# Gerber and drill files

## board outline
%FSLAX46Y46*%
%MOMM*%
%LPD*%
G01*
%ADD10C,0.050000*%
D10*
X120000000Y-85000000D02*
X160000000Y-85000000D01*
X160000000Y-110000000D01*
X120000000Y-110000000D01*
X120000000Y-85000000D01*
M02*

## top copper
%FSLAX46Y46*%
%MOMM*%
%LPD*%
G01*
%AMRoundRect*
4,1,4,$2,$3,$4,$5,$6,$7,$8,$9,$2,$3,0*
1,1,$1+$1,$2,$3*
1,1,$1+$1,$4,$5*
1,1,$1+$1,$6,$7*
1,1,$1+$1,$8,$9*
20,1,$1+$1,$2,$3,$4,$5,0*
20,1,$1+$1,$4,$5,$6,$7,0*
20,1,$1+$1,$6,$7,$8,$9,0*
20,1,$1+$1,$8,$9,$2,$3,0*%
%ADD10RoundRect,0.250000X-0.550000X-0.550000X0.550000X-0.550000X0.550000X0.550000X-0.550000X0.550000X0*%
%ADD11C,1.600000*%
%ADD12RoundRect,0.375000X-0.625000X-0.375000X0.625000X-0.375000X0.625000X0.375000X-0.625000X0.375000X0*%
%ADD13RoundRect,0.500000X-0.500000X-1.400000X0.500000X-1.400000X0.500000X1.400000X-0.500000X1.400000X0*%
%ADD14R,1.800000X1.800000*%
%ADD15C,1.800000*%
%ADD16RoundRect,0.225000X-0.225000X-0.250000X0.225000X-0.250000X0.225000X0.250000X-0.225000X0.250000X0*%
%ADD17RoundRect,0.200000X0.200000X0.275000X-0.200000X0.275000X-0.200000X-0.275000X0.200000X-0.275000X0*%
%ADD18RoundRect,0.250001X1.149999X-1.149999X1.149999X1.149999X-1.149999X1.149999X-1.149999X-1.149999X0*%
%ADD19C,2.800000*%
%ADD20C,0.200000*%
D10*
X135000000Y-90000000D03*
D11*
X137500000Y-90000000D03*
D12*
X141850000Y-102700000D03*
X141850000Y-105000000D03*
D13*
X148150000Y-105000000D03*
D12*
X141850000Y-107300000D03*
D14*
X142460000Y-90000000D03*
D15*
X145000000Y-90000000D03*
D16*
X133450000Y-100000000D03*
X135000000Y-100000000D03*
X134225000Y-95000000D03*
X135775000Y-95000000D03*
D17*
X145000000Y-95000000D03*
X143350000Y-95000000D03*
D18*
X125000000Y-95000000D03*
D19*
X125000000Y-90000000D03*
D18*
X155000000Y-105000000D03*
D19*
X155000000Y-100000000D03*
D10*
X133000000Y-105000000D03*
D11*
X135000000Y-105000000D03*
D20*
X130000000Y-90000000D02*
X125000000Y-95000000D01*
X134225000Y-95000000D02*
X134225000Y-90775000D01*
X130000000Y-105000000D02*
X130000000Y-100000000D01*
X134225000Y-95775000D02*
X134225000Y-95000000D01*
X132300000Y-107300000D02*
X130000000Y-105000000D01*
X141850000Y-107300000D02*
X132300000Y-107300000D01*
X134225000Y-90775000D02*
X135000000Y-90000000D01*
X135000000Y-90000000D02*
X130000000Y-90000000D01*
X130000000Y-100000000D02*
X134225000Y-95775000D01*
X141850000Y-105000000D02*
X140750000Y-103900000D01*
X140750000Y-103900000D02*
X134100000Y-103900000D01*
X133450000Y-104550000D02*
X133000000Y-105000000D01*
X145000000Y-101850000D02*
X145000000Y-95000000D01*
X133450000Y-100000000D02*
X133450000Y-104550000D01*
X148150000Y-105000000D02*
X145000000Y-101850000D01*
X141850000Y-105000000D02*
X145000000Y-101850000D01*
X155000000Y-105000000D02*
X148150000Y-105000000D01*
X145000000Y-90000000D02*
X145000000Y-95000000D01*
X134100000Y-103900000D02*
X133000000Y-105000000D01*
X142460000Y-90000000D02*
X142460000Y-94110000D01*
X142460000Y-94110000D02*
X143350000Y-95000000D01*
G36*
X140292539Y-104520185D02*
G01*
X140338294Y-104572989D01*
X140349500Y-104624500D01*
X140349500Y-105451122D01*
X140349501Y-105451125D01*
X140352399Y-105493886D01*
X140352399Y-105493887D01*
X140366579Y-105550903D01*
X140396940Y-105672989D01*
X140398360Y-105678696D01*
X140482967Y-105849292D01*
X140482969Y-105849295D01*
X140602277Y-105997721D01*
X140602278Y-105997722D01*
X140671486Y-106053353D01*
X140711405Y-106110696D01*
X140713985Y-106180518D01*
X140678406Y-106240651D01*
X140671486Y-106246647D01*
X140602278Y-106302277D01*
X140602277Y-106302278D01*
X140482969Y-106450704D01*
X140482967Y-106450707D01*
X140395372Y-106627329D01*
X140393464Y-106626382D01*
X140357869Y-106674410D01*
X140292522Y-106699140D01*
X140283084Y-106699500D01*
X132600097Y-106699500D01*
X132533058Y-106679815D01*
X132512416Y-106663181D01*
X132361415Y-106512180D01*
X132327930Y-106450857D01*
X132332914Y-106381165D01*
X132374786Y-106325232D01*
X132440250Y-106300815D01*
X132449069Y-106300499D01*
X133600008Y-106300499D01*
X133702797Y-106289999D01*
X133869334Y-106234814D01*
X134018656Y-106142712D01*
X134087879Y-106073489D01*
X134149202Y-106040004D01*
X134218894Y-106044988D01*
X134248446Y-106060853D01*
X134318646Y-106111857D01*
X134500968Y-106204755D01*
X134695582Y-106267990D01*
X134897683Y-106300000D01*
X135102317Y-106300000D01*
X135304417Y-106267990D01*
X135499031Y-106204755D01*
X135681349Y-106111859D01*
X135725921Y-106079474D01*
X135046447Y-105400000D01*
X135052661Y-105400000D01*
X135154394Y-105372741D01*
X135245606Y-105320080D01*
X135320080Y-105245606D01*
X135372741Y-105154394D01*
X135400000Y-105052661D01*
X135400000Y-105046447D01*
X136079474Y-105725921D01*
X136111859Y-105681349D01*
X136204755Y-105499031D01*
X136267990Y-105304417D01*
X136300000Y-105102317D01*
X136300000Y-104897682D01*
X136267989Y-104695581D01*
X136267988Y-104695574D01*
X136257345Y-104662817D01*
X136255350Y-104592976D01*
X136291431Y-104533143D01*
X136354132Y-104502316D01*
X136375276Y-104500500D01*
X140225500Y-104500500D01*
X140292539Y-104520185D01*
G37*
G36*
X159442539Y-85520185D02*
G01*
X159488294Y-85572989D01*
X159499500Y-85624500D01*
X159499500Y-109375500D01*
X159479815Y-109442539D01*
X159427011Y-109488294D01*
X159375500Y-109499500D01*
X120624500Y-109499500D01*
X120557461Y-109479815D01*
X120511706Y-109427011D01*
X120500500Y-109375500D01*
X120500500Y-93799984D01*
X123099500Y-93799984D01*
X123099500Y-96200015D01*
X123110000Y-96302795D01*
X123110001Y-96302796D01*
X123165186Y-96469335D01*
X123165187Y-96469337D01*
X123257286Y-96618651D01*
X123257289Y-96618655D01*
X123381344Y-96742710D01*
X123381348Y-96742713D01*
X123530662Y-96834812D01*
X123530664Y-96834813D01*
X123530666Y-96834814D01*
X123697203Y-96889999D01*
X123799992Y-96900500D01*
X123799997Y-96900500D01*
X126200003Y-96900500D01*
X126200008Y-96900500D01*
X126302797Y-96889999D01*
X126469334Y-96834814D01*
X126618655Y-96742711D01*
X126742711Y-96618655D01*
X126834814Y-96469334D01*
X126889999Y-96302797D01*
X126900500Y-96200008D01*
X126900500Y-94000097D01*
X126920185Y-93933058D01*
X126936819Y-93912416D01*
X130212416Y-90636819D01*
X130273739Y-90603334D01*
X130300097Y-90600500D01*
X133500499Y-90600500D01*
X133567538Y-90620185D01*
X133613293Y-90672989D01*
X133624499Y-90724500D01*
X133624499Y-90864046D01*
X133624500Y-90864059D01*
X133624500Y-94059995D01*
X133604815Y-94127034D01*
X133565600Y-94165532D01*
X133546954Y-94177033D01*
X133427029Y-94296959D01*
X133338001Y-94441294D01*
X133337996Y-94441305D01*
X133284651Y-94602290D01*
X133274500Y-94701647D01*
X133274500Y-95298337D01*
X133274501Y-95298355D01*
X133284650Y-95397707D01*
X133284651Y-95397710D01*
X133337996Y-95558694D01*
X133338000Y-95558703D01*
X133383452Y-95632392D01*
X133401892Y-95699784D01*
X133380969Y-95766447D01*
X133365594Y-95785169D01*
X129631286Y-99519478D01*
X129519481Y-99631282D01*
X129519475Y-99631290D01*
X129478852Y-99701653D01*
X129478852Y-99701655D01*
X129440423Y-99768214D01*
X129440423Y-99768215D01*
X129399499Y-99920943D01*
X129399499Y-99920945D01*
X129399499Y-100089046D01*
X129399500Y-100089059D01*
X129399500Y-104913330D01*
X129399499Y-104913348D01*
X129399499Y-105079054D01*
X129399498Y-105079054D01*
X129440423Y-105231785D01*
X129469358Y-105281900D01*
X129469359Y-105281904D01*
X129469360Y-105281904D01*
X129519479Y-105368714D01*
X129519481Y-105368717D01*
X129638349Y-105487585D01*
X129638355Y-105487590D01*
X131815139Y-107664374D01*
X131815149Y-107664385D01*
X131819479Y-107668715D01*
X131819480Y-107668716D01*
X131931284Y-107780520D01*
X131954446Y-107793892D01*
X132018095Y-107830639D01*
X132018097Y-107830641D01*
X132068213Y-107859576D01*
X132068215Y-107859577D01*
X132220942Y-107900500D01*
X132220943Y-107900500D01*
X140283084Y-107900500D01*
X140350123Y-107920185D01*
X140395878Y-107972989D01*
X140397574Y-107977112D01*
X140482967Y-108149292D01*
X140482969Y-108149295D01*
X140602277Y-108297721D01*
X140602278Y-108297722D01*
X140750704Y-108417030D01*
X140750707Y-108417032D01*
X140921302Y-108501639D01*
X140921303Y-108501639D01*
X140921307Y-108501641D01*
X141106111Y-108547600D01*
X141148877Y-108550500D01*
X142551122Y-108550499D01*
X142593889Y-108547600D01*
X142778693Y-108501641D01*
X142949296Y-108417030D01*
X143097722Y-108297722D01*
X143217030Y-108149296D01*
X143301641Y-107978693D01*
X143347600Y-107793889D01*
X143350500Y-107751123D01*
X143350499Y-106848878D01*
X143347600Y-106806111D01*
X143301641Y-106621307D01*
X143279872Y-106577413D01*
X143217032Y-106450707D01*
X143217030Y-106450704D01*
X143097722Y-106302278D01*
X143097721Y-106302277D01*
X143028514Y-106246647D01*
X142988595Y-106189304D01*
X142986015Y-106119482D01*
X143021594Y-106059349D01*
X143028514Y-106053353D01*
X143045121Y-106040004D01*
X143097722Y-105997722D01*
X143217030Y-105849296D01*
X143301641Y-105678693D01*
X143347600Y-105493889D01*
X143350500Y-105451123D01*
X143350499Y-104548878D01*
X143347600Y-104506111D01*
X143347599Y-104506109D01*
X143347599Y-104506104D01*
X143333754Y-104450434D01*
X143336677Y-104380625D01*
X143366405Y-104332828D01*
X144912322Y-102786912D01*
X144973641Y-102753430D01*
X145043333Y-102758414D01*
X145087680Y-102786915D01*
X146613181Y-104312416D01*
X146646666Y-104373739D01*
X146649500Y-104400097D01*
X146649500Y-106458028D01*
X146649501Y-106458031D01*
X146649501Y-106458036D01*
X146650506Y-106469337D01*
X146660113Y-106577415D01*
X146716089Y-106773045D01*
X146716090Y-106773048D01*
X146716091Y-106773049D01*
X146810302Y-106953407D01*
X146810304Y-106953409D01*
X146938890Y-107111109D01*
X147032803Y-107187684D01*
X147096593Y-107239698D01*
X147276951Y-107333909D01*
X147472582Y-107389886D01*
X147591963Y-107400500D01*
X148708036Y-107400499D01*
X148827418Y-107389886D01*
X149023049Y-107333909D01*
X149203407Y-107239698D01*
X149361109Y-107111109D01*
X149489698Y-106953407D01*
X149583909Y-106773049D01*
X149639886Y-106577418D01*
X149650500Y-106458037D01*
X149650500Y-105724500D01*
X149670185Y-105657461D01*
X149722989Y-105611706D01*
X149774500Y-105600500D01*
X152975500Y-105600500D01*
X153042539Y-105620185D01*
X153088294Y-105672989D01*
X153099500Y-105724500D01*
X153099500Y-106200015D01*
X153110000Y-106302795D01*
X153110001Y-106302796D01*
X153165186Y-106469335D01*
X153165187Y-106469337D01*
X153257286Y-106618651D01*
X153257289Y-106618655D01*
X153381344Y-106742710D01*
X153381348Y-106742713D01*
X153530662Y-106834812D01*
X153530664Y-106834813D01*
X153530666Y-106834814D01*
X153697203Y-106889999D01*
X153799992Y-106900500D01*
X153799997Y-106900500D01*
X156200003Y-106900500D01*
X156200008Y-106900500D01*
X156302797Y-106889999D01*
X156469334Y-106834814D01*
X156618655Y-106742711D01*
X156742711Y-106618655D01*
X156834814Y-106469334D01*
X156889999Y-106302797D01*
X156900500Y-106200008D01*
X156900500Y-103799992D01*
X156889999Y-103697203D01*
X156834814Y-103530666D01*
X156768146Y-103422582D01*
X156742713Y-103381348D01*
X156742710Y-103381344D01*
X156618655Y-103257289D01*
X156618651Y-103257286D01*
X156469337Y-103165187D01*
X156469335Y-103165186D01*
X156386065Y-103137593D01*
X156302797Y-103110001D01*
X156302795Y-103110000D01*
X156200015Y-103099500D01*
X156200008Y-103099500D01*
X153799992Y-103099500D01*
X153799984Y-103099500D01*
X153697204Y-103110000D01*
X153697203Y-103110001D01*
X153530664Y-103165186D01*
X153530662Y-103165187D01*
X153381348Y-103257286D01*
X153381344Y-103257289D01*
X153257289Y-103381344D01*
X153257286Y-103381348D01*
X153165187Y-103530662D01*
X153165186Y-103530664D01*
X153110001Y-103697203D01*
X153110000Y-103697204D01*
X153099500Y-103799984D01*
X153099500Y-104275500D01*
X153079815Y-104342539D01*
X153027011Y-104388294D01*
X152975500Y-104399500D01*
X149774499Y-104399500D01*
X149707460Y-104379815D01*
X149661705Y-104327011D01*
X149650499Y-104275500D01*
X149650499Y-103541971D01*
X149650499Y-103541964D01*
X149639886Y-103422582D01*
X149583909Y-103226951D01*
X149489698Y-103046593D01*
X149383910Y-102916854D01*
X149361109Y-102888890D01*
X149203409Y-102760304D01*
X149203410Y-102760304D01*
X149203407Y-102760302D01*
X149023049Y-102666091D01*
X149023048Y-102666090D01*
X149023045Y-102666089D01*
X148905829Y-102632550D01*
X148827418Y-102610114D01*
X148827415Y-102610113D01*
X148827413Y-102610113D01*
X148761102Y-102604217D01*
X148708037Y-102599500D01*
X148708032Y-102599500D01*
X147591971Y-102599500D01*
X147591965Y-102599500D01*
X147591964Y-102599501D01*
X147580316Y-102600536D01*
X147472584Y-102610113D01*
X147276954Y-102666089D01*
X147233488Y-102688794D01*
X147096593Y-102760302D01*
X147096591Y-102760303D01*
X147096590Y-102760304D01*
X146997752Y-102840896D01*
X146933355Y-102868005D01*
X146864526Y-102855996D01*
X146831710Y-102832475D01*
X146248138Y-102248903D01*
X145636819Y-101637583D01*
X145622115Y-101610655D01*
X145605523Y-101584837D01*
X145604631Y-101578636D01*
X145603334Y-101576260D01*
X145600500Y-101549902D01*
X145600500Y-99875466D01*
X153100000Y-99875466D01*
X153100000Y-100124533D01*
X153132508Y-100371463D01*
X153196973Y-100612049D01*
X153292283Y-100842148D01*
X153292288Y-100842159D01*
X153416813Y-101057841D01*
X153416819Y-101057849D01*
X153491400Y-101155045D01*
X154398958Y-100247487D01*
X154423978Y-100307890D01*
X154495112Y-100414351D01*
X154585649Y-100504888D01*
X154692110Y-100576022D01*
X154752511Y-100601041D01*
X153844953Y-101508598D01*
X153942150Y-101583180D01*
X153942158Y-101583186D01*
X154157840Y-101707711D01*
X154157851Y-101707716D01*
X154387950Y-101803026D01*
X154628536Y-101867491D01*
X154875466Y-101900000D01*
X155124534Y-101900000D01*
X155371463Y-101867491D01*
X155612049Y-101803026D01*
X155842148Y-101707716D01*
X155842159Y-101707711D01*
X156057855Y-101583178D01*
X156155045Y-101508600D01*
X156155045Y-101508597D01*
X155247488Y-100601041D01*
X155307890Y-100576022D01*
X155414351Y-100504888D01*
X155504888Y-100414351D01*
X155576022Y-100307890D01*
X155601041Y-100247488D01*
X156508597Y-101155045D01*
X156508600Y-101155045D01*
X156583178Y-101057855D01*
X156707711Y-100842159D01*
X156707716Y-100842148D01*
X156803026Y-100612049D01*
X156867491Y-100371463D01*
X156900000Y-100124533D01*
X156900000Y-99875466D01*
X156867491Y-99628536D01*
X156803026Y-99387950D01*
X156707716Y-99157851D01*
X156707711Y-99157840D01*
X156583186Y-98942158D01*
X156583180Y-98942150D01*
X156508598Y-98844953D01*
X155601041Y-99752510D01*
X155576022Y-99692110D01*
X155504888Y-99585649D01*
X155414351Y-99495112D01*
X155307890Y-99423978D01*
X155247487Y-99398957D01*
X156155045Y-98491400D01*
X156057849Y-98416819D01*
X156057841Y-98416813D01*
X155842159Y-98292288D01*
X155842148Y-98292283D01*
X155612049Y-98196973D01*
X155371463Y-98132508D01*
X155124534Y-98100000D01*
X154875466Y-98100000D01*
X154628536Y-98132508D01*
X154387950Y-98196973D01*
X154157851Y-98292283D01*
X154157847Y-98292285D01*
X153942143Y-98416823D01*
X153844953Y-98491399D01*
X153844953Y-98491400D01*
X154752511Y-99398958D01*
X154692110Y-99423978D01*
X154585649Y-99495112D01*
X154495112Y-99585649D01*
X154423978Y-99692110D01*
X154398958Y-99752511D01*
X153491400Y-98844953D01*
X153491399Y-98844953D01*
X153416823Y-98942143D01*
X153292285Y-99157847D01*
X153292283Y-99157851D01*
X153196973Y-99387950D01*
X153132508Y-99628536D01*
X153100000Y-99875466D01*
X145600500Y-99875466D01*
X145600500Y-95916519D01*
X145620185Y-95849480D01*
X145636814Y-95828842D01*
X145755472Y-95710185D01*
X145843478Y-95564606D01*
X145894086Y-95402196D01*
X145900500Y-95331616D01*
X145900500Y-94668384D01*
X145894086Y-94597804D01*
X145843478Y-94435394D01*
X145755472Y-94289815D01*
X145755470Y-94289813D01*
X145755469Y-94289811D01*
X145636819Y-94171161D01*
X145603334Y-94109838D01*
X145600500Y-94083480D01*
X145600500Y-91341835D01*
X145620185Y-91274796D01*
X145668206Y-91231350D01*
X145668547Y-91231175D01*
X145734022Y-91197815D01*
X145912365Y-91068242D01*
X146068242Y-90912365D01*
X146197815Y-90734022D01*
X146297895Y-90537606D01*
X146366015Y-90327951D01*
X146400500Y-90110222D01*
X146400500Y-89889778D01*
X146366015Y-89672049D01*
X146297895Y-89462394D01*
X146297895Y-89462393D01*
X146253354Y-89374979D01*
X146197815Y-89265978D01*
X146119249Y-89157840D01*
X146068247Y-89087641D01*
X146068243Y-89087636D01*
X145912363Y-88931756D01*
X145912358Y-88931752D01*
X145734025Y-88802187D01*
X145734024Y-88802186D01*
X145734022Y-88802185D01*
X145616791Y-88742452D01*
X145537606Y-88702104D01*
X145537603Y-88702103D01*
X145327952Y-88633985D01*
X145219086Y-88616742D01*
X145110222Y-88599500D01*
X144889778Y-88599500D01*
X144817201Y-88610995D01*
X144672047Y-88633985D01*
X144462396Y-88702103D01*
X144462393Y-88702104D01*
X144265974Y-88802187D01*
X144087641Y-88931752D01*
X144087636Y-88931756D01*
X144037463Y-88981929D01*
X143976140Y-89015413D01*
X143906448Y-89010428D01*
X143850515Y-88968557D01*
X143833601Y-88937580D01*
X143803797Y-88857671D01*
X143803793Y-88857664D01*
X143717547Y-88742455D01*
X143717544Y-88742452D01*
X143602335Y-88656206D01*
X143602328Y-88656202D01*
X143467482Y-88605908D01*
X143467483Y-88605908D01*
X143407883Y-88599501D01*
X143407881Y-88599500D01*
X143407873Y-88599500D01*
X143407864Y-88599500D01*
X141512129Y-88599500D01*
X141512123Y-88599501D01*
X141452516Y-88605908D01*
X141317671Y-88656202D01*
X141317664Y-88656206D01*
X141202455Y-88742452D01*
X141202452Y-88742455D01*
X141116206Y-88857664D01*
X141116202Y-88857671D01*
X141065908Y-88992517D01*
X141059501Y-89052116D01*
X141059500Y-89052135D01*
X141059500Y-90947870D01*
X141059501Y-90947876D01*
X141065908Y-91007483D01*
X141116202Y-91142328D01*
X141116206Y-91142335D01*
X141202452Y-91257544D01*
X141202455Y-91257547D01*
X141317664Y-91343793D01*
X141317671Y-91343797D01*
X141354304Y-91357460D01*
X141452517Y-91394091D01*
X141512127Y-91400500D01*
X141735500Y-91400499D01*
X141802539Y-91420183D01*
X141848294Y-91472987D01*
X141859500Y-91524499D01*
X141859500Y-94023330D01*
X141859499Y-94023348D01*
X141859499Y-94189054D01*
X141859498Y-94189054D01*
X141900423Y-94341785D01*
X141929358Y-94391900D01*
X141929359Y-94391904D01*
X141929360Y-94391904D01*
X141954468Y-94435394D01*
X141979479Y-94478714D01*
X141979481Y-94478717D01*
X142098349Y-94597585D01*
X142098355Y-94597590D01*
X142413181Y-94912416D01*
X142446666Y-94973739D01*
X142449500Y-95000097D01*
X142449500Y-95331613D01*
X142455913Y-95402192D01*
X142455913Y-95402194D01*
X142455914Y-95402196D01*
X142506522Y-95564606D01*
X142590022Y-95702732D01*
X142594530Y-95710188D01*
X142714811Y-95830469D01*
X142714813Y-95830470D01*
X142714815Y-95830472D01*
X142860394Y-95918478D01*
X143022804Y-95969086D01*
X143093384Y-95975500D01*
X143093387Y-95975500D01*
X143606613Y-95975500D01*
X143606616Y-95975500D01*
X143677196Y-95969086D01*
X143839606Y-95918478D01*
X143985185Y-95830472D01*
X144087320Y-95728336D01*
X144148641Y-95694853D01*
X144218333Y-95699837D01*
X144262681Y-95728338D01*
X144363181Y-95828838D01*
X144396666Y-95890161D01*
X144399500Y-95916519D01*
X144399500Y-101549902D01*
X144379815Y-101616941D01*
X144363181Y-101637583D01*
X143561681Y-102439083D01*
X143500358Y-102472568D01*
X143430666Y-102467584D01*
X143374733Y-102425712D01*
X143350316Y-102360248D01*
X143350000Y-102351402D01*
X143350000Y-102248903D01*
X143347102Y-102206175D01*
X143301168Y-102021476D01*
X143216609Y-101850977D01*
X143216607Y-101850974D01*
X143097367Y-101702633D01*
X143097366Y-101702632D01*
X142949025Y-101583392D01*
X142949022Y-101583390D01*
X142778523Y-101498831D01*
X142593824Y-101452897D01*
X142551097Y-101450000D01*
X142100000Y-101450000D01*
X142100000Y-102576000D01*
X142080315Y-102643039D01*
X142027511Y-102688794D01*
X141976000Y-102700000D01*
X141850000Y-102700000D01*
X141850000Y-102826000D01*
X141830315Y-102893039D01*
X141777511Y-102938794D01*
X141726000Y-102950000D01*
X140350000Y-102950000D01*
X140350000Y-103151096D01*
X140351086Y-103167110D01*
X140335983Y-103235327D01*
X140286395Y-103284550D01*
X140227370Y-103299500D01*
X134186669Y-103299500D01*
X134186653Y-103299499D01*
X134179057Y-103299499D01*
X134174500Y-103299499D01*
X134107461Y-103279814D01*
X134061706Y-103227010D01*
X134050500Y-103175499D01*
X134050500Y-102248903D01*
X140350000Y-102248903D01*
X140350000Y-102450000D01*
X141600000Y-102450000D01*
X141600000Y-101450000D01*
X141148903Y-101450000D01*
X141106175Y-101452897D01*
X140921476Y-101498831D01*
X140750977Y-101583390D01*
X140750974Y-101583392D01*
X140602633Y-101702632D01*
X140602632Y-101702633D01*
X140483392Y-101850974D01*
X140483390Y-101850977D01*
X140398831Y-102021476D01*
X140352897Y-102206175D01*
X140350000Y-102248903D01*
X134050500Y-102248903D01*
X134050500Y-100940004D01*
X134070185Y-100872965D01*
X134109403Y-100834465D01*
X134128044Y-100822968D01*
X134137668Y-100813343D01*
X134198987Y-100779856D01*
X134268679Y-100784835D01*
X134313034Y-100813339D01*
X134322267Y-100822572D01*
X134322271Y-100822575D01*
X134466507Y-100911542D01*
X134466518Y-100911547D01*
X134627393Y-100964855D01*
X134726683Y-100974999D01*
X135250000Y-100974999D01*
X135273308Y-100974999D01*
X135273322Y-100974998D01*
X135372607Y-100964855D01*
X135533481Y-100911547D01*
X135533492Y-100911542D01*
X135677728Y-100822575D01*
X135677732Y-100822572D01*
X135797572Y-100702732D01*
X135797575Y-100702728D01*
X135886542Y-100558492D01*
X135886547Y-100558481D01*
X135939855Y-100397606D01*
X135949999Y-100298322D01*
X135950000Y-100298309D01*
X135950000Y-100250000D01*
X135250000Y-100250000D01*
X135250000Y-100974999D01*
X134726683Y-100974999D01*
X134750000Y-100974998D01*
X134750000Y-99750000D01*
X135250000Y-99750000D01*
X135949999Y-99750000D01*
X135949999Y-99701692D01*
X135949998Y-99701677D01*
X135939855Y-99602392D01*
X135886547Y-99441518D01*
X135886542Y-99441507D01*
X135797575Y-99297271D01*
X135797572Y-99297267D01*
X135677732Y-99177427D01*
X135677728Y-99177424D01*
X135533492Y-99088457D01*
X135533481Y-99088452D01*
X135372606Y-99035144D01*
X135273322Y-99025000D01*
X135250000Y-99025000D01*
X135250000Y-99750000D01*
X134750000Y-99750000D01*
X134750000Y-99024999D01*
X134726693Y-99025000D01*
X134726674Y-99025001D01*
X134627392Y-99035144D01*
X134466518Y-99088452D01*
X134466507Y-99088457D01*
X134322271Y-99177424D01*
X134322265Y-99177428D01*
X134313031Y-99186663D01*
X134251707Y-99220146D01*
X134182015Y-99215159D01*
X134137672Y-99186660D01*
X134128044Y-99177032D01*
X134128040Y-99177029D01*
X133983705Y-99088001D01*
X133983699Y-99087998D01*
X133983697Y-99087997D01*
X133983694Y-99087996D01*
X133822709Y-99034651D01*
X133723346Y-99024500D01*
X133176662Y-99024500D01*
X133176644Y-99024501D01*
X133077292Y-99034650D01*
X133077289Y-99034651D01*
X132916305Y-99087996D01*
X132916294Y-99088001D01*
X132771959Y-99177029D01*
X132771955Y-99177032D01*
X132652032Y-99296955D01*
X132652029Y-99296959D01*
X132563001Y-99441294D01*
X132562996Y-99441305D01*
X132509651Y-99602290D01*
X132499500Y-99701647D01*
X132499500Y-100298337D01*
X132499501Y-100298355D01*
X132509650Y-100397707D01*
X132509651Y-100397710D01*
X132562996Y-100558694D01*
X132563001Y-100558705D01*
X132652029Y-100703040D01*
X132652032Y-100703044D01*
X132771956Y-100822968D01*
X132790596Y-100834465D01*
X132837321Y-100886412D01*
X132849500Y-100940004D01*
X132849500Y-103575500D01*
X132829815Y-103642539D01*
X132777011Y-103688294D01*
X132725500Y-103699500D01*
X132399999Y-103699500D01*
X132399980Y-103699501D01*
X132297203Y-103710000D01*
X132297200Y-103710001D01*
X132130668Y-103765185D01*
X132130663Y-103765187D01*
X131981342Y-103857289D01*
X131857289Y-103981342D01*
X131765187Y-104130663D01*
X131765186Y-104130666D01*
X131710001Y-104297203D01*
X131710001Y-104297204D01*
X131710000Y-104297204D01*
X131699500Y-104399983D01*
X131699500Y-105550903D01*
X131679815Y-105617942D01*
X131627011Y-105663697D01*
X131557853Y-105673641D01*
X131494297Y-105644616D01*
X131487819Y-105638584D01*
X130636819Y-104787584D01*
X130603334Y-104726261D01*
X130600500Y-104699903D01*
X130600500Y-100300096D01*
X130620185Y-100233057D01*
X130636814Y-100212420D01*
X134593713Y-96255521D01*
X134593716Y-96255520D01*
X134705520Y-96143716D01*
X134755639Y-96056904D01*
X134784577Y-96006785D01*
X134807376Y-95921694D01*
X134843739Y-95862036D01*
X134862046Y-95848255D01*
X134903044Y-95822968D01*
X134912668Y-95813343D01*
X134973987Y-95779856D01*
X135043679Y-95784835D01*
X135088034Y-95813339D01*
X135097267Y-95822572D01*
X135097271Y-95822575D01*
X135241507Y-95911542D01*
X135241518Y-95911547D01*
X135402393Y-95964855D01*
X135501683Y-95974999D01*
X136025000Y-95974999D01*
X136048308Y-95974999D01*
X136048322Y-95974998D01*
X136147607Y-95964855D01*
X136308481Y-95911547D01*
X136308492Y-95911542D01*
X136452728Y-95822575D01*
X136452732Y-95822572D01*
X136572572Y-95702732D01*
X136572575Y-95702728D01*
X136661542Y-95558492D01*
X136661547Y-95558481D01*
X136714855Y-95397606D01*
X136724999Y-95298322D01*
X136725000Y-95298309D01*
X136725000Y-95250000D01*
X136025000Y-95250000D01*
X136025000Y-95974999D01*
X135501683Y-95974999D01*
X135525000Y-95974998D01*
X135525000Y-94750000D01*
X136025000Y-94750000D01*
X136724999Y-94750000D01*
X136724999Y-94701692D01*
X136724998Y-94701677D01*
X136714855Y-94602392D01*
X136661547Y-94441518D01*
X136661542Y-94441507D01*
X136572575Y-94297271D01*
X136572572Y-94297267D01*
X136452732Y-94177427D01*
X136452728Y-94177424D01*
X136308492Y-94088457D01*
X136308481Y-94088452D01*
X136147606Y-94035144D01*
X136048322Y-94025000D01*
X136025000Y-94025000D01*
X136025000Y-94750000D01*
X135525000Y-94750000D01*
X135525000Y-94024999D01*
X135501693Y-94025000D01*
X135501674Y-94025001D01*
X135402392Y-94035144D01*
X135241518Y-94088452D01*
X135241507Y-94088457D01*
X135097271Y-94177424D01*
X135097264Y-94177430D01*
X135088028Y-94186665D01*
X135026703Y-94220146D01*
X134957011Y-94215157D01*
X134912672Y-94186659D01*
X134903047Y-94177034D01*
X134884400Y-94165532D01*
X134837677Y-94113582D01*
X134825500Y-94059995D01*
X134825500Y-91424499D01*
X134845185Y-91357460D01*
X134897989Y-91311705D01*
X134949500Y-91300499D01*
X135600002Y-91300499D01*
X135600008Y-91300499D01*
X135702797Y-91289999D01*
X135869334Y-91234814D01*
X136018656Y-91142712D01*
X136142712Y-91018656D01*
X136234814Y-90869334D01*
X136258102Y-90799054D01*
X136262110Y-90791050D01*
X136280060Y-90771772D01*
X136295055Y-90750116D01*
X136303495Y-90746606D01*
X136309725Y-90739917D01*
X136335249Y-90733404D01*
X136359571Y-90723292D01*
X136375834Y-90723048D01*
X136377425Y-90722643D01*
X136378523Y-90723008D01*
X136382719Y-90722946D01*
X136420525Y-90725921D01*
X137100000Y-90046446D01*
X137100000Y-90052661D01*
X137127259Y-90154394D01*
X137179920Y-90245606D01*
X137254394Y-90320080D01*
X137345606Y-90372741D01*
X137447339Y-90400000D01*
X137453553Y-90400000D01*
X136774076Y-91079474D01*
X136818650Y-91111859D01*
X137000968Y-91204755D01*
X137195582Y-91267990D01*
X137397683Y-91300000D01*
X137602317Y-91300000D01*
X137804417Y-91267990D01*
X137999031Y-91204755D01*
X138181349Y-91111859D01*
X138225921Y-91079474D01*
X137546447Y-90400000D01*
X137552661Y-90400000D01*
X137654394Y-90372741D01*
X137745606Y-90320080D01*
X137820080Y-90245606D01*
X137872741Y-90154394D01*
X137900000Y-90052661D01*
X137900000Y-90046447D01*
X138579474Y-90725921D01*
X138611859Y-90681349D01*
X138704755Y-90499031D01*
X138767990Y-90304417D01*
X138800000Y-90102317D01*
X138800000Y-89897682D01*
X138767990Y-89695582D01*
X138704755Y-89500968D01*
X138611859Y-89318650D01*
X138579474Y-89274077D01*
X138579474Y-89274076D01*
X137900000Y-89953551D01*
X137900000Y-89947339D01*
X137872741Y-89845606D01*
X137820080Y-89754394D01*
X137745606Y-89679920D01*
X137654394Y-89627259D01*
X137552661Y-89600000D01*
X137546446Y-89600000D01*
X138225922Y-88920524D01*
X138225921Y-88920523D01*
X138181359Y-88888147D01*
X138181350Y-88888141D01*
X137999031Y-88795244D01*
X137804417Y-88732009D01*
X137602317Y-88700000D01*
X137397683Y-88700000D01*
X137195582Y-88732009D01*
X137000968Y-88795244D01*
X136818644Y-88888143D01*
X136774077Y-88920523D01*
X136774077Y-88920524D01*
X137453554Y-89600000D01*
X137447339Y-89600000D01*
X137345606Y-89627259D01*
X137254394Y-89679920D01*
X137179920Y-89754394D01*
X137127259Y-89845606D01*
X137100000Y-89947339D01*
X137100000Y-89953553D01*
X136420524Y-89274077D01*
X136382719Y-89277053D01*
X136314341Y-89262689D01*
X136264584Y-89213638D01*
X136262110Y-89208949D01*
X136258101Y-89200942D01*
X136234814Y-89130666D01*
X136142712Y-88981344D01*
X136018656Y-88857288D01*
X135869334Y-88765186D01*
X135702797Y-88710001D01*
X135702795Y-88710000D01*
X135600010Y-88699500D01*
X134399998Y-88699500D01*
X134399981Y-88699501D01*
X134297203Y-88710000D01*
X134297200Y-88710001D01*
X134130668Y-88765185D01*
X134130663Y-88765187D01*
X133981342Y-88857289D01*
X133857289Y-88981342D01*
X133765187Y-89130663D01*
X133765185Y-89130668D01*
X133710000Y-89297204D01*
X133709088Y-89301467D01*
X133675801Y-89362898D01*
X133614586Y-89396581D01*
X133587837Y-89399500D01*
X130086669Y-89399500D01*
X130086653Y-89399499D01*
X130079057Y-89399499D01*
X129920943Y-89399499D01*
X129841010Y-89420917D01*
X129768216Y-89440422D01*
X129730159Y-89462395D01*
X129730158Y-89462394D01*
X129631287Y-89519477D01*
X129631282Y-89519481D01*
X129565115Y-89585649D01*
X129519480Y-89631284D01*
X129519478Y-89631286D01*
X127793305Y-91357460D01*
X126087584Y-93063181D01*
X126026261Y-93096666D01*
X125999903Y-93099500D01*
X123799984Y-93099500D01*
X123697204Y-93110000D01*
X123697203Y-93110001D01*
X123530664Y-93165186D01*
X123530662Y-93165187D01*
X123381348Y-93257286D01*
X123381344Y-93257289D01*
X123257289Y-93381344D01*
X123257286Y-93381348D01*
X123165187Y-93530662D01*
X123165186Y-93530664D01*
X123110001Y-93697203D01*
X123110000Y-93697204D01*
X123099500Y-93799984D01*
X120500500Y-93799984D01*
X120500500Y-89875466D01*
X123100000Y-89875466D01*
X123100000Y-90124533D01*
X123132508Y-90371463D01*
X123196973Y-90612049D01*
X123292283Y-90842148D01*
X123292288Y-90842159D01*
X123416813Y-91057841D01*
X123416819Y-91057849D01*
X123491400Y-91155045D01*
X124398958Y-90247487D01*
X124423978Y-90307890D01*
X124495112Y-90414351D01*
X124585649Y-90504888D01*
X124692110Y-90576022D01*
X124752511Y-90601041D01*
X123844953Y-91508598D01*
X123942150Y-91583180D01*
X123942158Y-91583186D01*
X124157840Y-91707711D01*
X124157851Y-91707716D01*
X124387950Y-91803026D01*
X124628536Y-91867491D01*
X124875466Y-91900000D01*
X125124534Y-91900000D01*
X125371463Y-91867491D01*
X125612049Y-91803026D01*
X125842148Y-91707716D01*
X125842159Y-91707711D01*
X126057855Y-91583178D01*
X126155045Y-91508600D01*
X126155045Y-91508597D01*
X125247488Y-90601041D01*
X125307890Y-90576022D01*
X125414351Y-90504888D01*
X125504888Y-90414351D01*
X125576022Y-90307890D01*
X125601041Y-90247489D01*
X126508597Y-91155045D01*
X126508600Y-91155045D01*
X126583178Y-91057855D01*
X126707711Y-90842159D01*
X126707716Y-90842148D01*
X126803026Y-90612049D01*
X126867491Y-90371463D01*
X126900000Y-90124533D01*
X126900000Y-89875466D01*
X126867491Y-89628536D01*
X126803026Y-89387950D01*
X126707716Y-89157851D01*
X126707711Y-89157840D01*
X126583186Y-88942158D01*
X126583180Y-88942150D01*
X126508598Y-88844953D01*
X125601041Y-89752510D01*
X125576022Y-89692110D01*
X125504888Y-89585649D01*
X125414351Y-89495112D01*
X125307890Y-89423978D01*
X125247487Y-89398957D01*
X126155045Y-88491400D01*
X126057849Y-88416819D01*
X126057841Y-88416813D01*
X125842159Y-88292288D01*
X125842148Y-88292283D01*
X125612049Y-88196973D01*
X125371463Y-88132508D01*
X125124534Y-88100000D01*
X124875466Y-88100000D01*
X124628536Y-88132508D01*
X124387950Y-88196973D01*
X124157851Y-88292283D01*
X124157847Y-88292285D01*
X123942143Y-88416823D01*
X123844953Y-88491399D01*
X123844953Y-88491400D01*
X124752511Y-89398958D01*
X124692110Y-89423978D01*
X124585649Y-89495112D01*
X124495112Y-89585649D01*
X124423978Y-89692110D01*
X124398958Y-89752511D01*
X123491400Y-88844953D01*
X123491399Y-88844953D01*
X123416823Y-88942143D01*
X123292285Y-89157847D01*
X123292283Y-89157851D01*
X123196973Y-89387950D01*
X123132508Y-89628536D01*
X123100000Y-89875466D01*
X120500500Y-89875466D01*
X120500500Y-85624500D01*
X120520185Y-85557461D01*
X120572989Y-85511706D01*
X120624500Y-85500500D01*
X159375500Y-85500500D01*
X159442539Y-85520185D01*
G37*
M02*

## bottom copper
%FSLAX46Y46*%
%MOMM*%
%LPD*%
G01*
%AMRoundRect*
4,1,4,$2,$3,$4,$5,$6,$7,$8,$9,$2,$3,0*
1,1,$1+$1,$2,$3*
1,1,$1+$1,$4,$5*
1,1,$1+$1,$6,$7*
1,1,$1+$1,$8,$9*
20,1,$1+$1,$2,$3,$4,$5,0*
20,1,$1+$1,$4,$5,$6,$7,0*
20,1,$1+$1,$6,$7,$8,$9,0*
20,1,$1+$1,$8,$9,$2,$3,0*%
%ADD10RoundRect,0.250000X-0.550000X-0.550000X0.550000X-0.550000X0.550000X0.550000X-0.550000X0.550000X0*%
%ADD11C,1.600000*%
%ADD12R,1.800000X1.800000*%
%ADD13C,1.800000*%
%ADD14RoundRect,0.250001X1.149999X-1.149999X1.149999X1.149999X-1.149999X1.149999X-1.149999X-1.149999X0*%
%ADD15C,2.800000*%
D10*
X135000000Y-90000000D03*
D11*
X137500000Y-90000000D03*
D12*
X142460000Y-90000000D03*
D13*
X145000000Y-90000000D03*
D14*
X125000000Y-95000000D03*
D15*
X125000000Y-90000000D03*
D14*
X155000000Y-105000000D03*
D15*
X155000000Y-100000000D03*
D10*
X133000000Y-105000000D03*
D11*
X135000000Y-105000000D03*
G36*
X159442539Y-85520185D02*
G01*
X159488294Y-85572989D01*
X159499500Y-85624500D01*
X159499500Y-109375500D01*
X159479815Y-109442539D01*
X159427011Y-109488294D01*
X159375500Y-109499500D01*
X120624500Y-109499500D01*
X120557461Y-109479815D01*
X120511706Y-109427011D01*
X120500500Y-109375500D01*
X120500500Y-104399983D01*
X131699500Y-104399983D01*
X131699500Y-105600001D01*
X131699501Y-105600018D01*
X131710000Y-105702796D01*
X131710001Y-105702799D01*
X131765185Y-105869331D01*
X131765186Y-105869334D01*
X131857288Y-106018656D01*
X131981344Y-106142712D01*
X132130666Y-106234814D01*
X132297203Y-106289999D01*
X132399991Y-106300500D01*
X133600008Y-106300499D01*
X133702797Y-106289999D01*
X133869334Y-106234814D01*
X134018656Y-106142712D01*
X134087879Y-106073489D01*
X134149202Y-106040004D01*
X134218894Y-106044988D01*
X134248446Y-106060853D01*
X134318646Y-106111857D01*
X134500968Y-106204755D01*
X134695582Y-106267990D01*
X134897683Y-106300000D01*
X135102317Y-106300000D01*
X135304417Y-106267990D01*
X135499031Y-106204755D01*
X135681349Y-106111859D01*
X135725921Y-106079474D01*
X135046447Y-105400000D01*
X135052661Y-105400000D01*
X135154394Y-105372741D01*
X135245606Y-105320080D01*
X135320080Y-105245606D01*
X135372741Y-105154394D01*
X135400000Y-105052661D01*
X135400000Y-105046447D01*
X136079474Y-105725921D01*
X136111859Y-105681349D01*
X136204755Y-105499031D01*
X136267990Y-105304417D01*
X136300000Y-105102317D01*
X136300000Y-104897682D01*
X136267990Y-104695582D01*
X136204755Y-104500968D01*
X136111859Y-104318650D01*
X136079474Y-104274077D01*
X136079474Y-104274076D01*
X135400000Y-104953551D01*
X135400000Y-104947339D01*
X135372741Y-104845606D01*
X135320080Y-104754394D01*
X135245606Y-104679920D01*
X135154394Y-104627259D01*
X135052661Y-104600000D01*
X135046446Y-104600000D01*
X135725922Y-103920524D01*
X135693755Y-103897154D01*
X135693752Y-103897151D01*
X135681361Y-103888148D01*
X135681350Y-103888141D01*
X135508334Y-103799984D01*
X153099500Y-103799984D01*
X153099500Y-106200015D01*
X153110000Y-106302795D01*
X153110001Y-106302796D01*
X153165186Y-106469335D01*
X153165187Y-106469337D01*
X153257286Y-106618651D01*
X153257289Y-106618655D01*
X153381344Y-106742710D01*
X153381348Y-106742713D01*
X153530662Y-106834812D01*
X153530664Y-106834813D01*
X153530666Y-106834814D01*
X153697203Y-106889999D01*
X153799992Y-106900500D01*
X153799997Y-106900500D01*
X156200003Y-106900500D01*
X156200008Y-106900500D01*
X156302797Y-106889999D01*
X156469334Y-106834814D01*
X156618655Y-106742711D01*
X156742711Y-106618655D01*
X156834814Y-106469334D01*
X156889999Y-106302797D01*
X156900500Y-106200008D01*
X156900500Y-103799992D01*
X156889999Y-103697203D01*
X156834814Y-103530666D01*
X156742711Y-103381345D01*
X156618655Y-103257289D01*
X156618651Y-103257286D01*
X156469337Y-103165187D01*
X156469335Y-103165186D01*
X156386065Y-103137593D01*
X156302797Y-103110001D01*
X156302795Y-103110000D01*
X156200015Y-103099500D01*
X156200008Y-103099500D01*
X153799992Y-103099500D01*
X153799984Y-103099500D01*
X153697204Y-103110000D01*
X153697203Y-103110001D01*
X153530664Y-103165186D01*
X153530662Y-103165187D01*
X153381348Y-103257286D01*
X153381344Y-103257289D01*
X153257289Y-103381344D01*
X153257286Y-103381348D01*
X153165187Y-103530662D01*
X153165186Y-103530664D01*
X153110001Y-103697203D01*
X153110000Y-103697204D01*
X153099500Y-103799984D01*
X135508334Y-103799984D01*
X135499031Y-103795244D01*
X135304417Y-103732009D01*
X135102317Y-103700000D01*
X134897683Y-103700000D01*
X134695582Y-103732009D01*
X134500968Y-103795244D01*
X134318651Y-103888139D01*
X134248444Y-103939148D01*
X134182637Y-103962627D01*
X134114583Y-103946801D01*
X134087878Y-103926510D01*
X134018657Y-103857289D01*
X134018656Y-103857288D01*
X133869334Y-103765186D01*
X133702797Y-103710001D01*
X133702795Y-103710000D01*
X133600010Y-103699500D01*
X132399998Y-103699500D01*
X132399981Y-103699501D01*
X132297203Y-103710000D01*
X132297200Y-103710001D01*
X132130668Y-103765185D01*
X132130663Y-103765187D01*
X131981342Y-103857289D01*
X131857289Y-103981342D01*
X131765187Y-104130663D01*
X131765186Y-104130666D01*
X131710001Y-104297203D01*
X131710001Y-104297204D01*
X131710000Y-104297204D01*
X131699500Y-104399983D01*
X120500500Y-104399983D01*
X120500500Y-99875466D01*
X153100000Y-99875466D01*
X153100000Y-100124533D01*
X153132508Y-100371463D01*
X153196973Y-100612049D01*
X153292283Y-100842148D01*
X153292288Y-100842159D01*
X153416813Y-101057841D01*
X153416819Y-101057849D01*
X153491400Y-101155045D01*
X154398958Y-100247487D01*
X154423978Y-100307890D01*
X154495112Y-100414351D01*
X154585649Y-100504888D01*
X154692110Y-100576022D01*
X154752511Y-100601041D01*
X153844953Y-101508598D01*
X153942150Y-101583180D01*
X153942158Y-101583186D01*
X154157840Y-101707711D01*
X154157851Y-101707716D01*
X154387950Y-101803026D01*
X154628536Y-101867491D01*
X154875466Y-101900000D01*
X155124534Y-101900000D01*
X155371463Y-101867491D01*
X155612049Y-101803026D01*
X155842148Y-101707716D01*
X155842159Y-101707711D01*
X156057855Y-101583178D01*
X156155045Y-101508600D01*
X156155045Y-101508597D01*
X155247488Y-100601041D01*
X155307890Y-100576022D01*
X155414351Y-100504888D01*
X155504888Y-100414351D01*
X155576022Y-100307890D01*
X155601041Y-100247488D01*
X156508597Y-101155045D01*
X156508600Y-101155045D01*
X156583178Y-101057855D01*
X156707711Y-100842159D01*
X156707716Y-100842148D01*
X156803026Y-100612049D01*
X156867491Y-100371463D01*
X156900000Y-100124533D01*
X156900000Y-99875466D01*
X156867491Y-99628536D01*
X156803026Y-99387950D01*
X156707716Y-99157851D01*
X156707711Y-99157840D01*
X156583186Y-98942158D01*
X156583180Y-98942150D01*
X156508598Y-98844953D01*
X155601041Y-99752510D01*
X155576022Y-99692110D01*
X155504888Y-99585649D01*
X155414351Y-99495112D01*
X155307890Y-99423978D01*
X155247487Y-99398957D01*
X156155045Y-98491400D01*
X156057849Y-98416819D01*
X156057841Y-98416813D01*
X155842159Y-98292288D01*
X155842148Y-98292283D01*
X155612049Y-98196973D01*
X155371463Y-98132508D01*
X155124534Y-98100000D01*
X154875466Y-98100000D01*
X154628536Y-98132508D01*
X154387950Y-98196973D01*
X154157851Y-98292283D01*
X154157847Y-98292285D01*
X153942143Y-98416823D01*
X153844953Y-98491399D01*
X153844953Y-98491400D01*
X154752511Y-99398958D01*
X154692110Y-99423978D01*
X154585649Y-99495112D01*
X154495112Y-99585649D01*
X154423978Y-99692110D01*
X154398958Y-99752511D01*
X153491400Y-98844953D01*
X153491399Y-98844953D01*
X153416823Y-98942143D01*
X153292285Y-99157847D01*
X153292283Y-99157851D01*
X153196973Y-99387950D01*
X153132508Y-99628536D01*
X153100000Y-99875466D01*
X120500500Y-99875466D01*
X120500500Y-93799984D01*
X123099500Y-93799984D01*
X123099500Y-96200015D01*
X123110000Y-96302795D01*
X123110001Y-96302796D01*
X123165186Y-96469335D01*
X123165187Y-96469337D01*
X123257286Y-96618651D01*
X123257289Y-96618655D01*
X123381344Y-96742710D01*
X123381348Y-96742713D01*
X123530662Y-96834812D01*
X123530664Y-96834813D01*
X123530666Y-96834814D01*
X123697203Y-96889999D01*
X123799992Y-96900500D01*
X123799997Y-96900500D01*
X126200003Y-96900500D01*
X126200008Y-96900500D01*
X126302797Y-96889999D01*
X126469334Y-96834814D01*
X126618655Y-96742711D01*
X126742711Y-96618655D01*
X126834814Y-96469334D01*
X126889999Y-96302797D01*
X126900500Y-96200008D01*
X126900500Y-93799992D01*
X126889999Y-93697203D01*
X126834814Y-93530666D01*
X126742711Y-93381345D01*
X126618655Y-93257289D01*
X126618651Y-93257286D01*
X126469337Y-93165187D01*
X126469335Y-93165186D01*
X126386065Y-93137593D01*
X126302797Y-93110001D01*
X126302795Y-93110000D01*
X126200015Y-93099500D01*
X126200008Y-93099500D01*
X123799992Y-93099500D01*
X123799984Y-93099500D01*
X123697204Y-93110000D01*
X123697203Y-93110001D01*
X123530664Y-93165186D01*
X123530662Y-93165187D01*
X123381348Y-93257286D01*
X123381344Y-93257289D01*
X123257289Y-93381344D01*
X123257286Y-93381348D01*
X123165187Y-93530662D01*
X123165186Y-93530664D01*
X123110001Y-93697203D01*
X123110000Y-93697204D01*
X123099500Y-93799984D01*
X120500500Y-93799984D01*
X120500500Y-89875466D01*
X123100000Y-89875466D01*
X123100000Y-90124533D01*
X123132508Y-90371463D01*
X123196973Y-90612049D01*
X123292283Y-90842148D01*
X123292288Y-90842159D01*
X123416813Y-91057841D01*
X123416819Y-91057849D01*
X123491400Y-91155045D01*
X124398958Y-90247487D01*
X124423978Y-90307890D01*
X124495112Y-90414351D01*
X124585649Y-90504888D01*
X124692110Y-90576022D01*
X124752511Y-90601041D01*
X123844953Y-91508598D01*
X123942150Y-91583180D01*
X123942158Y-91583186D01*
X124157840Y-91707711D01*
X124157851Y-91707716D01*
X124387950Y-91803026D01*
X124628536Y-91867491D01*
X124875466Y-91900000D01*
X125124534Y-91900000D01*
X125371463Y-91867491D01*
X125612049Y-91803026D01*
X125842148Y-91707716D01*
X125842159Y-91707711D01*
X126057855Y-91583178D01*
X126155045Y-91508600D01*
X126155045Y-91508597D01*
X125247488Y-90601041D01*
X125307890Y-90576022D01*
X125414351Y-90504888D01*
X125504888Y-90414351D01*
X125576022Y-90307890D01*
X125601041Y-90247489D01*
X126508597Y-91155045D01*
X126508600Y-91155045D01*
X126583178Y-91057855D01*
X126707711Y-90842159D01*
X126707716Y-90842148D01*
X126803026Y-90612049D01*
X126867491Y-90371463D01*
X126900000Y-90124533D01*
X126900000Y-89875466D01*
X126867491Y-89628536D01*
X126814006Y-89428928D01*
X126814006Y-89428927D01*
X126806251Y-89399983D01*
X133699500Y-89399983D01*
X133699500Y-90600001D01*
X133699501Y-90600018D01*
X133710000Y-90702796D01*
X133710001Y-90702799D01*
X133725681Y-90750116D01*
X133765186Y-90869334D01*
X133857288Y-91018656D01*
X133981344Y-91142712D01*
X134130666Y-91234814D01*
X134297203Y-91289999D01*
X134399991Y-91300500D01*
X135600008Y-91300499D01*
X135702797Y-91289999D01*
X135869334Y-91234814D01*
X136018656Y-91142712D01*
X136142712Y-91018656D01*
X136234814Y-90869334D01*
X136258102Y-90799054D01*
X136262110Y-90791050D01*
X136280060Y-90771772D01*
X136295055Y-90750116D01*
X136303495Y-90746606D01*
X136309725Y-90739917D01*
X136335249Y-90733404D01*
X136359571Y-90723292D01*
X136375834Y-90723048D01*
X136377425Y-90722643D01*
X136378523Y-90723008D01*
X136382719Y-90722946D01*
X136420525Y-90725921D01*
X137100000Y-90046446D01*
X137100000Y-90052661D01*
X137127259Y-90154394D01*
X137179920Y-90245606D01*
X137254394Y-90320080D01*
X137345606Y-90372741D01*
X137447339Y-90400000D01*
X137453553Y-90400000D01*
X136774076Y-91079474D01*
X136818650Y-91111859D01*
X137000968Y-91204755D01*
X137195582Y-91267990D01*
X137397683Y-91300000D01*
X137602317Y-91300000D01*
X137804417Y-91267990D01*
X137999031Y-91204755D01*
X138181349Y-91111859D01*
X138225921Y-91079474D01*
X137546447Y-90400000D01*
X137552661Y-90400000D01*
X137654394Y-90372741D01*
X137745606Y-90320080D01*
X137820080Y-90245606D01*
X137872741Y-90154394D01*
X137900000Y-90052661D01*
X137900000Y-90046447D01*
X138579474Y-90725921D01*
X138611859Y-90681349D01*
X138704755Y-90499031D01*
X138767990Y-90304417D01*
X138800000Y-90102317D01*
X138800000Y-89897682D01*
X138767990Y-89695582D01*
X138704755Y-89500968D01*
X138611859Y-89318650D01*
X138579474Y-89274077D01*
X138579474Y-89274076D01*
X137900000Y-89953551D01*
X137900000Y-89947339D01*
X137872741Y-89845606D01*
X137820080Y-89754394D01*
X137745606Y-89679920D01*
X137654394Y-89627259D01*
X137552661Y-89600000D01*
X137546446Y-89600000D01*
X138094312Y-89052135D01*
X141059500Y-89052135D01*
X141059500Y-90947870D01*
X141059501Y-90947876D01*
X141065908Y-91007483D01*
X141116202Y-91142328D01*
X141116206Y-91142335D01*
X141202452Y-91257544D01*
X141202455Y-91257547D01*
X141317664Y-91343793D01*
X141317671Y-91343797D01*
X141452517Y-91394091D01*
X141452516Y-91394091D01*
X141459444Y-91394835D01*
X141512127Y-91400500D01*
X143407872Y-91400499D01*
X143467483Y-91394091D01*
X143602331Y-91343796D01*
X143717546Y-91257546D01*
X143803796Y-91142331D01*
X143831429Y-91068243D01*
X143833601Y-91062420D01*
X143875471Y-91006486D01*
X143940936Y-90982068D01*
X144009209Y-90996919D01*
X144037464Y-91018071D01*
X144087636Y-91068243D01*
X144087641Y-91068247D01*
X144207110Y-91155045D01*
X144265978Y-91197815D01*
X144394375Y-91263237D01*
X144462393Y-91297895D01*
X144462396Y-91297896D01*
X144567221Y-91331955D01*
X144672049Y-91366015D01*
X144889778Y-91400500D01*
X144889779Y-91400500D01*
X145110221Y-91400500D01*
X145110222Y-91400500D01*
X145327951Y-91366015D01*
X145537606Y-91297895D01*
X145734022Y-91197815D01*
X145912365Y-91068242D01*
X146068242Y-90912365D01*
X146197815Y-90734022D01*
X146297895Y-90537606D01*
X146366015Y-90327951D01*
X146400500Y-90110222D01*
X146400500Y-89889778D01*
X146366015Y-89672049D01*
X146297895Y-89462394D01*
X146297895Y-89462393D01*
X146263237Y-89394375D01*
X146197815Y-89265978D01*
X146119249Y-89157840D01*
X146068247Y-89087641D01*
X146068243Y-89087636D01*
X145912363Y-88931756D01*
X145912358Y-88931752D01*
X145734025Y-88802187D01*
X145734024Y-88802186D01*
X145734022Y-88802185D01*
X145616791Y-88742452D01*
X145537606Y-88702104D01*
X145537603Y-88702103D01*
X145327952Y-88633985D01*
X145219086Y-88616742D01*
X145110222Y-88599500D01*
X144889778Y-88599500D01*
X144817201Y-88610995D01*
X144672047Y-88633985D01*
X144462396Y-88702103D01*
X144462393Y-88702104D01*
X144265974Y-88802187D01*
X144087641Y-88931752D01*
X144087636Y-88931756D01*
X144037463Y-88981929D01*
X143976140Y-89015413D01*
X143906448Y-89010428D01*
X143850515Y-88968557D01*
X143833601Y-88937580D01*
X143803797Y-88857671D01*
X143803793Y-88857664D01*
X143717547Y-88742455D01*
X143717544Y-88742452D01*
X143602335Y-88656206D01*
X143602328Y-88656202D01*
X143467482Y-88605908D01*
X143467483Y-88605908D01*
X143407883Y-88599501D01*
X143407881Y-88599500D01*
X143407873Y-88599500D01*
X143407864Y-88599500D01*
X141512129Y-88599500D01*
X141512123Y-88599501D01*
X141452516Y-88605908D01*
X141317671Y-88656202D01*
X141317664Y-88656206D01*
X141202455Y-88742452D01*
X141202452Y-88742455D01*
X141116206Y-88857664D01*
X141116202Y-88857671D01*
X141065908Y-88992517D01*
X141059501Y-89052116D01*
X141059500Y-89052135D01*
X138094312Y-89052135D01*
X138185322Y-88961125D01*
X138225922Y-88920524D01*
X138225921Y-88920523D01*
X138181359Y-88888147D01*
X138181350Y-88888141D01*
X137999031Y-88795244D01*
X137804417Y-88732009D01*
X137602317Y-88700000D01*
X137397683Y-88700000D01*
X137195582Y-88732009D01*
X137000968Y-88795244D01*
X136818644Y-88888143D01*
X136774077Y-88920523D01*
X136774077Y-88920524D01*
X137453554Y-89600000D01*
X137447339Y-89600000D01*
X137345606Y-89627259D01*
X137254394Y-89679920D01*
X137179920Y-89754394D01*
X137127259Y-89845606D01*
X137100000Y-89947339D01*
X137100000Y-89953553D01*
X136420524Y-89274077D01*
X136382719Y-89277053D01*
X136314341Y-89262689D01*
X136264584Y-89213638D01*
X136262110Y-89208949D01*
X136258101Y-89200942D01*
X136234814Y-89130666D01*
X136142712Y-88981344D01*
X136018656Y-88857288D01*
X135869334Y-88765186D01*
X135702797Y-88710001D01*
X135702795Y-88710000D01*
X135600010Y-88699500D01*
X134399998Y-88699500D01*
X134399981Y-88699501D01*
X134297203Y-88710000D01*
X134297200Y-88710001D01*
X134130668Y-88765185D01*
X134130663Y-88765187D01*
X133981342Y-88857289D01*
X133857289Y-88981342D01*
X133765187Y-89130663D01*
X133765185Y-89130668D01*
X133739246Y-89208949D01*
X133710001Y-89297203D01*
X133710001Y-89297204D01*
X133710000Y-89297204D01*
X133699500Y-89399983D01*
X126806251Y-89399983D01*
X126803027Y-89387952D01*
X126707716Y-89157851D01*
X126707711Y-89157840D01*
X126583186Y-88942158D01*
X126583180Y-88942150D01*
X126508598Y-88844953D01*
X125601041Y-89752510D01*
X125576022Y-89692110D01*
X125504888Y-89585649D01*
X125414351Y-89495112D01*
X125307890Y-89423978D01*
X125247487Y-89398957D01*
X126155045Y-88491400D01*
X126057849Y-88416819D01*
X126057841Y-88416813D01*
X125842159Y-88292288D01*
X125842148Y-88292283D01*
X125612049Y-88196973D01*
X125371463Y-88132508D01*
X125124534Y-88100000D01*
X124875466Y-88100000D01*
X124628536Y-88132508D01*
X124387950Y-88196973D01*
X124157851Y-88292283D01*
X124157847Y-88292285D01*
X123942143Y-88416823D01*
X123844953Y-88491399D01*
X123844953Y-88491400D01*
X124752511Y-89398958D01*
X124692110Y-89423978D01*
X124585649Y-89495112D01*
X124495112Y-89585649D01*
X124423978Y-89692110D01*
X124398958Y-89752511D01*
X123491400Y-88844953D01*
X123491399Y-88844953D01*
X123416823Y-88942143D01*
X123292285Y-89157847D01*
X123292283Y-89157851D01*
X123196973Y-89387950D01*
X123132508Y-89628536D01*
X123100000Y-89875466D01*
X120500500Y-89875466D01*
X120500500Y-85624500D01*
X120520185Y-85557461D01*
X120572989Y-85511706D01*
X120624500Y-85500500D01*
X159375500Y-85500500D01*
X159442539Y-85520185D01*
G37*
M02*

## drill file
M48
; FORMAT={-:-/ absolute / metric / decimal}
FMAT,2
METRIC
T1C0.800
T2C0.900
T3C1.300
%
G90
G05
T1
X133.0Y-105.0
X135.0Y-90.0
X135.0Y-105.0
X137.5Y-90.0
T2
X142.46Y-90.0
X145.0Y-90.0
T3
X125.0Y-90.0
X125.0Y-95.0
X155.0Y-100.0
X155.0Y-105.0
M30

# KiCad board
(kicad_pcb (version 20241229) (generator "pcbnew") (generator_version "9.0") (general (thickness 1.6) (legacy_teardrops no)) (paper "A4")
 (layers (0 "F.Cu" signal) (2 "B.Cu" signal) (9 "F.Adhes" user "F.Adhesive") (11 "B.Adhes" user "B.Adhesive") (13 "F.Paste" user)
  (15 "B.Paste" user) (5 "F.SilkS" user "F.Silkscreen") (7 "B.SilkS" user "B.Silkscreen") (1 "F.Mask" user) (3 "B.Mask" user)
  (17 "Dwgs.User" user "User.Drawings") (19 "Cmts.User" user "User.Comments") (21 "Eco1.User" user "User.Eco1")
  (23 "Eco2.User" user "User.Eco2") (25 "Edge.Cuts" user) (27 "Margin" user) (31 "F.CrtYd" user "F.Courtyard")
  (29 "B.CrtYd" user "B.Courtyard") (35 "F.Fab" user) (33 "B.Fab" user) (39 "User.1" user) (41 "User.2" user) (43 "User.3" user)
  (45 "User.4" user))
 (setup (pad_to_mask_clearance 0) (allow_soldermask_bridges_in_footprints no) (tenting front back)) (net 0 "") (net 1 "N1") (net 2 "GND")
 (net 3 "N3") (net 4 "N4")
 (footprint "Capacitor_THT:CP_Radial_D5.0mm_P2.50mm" (layer "F.Cu") (at 135 90)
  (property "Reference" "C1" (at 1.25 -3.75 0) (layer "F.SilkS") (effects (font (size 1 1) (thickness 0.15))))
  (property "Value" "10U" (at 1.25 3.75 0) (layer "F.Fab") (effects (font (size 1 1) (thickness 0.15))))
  (pad "1" thru_hole roundrect (at 0 0) (size 1.6 1.6) (drill 0.8) (layers "*.Cu" "*.Mask") (remove_unused_layers no)
   (roundrect_rratio 0.15625) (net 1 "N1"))
  (pad "2" thru_hole circle (at 2.5 0) (size 1.6 1.6) (drill 0.8) (layers "*.Cu" "*.Mask") (remove_unused_layers no) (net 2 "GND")))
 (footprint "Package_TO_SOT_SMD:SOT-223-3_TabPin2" (layer "F.Cu") (at 145 105)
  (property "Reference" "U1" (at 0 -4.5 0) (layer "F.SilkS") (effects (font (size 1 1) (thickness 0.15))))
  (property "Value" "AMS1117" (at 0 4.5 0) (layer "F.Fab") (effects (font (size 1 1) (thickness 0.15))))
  (pad "1" smd roundrect (at -3.15 -2.3) (size 2 1.5) (layers "F.Cu" "F.Mask" "F.Paste") (roundrect_rratio 0.25) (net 2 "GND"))
  (pad "2" smd roundrect (at -3.15 0) (size 2 1.5) (layers "F.Cu" "F.Mask" "F.Paste") (roundrect_rratio 0.25) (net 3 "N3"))
  (pad "2" smd roundrect (at 3.15 0) (size 2 3.8) (layers "F.Cu" "F.Mask" "F.Paste") (roundrect_rratio 0.25) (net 3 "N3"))
  (pad "3" smd roundrect (at -3.15 2.3) (size 2 1.5) (layers "F.Cu" "F.Mask" "F.Paste") (roundrect_rratio 0.25) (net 1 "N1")))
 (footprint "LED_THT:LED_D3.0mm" (layer "F.Cu") (at 142.46 90)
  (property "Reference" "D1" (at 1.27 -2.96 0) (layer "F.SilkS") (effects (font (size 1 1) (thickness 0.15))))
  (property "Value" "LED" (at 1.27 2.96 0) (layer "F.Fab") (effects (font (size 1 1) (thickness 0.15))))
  (pad "1" thru_hole rect (at 0 0) (size 1.8 1.8) (drill 0.9) (layers "*.Cu" "*.Mask") (remove_unused_layers no) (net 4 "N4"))
  (pad "2" thru_hole circle (at 2.54 0) (size 1.8 1.8) (drill 0.9) (layers "*.Cu" "*.Mask") (remove_unused_layers no) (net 3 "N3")))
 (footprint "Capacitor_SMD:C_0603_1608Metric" (layer "F.Cu") (at 134.225 100)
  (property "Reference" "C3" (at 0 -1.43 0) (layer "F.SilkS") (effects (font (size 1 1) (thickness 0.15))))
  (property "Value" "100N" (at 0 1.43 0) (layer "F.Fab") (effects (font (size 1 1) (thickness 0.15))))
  (pad "1" smd roundrect (at -0.775 0) (size 0.9 0.95) (layers "F.Cu" "F.Mask" "F.Paste") (roundrect_rratio 0.25) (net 3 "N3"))
  (pad "2" smd roundrect (at 0.775 0) (size 0.9 0.95) (layers "F.Cu" "F.Mask" "F.Paste") (roundrect_rratio 0.25) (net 2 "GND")))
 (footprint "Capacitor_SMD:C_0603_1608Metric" (layer "F.Cu") (at 135 95)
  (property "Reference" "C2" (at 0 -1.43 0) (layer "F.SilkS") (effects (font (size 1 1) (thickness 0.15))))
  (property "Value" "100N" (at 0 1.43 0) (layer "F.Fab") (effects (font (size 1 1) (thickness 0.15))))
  (pad "1" smd roundrect (at -0.775 0) (size 0.9 0.95) (layers "F.Cu" "F.Mask" "F.Paste") (roundrect_rratio 0.25) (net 1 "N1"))
  (pad "2" smd roundrect (at 0.775 0) (size 0.9 0.95) (layers "F.Cu" "F.Mask" "F.Paste") (roundrect_rratio 0.25) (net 2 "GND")))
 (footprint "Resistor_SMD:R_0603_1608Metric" (layer "F.Cu") (at 144.175 95 180)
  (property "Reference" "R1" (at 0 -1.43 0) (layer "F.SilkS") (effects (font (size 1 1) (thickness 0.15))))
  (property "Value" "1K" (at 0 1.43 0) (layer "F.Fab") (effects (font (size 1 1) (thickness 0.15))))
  (pad "1" smd roundrect (at -0.825 0 180) (size 0.8 0.95) (layers "F.Cu" "F.Mask" "F.Paste") (roundrect_rratio 0.25) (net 3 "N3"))
  (pad "2" smd roundrect (at 0.825 0 180) (size 0.8 0.95) (layers "F.Cu" "F.Mask" "F.Paste") (roundrect_rratio 0.25) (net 4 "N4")))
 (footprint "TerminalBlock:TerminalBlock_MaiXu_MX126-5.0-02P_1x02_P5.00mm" (layer "F.Cu") (at 125 95 90)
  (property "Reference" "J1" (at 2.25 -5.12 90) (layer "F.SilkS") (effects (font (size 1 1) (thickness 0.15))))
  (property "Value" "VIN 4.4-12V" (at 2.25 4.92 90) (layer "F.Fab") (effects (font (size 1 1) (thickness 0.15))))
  (pad "1" thru_hole roundrect (at 0 0 90) (size 2.8 2.8) (drill 1.3) (layers "*.Cu" "*.Mask") (remove_unused_layers no)
   (roundrect_rratio 0.089286) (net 1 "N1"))
  (pad "2" thru_hole circle (at 5 0 90) (size 2.8 2.8) (drill 1.3) (layers "*.Cu" "*.Mask") (remove_unused_layers no) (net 2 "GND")))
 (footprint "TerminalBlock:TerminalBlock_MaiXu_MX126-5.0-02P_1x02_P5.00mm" (layer "F.Cu") (at 155 105 90)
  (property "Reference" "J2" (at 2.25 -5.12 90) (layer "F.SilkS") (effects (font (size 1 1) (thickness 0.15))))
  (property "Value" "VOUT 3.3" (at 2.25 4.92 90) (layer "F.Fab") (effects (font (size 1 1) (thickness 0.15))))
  (pad "1" thru_hole roundrect (at 0 0 90) (size 2.8 2.8) (drill 1.3) (layers "*.Cu" "*.Mask") (remove_unused_layers no)
   (roundrect_rratio 0.089286) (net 3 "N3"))
  (pad "2" thru_hole circle (at 5 0 90) (size 2.8 2.8) (drill 1.3) (layers "*.Cu" "*.Mask") (remove_unused_layers no) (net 2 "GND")))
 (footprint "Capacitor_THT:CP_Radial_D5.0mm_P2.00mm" (layer "F.Cu") (at 133 105)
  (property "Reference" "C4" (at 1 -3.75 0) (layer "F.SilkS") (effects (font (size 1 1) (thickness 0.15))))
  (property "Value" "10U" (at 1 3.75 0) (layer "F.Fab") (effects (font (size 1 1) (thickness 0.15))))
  (pad "1" thru_hole roundrect (at 0 0) (size 1.6 1.6) (drill 0.8) (layers "*.Cu" "*.Mask") (remove_unused_layers no)
   (roundrect_rratio 0.15625) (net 3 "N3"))
  (pad "2" thru_hole circle (at 2 0) (size 1.6 1.6) (drill 0.8) (layers "*.Cu" "*.Mask") (remove_unused_layers no) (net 2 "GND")))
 (gr_rect (start 120 85) (end 160 110) (stroke (width 0.05) (type default)) (fill no) (layer "Edge.Cuts"))
 (segment (start 130 90) (end 125 95) (width 0.2) (layer "F.Cu") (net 1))
 (segment (start 134.225 95) (end 134.225 90.775) (width 0.2) (layer "F.Cu") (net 1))
 (segment (start 130 105) (end 130 100) (width 0.2) (layer "F.Cu") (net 1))
 (segment (start 134.225 95.775) (end 134.225 95) (width 0.2) (layer "F.Cu") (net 1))
 (segment (start 132.3 107.3) (end 130 105) (width 0.2) (layer "F.Cu") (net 1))
 (segment (start 141.85 107.3) (end 132.3 107.3) (width 0.2) (layer "F.Cu") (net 1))
 (segment (start 134.225 90.775) (end 135 90) (width 0.2) (layer "F.Cu") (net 1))
 (segment (start 135 90) (end 130 90) (width 0.2) (layer "F.Cu") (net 1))
 (segment (start 130 100) (end 134.225 95.775) (width 0.2) (layer "F.Cu") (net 1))
 (segment (start 141.85 105) (end 140.75 103.9) (width 0.2) (layer "F.Cu") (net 3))
 (segment (start 140.75 103.9) (end 134.1 103.9) (width 0.2) (layer "F.Cu") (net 3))
 (segment (start 133.45 104.55) (end 133 105) (width 0.2) (layer "F.Cu") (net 3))
 (segment (start 145 101.85) (end 145 95) (width 0.2) (layer "F.Cu") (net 3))
 (segment (start 133.45 100) (end 133.45 104.55) (width 0.2) (layer "F.Cu") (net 3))
 (segment (start 148.15 105) (end 145 101.85) (width 0.2) (layer "F.Cu") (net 3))
 (segment (start 141.85 105) (end 145 101.85) (width 0.2) (layer "F.Cu") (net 3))
 (segment (start 155 105) (end 148.15 105) (width 0.2) (layer "F.Cu") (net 3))
 (segment (start 145 90) (end 145 95) (width 0.2) (layer "F.Cu") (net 3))
 (segment (start 134.1 103.9) (end 133 105) (width 0.2) (layer "F.Cu") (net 3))
 (segment (start 142.46 90) (end 142.46 94.11) (width 0.2) (layer "F.Cu") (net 4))
 (segment (start 142.46 94.11) (end 143.35 95) (width 0.2) (layer "F.Cu") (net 4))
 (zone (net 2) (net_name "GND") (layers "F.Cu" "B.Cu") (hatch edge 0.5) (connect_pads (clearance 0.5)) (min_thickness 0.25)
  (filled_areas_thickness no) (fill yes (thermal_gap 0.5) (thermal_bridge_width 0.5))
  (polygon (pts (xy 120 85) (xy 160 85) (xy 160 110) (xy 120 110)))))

